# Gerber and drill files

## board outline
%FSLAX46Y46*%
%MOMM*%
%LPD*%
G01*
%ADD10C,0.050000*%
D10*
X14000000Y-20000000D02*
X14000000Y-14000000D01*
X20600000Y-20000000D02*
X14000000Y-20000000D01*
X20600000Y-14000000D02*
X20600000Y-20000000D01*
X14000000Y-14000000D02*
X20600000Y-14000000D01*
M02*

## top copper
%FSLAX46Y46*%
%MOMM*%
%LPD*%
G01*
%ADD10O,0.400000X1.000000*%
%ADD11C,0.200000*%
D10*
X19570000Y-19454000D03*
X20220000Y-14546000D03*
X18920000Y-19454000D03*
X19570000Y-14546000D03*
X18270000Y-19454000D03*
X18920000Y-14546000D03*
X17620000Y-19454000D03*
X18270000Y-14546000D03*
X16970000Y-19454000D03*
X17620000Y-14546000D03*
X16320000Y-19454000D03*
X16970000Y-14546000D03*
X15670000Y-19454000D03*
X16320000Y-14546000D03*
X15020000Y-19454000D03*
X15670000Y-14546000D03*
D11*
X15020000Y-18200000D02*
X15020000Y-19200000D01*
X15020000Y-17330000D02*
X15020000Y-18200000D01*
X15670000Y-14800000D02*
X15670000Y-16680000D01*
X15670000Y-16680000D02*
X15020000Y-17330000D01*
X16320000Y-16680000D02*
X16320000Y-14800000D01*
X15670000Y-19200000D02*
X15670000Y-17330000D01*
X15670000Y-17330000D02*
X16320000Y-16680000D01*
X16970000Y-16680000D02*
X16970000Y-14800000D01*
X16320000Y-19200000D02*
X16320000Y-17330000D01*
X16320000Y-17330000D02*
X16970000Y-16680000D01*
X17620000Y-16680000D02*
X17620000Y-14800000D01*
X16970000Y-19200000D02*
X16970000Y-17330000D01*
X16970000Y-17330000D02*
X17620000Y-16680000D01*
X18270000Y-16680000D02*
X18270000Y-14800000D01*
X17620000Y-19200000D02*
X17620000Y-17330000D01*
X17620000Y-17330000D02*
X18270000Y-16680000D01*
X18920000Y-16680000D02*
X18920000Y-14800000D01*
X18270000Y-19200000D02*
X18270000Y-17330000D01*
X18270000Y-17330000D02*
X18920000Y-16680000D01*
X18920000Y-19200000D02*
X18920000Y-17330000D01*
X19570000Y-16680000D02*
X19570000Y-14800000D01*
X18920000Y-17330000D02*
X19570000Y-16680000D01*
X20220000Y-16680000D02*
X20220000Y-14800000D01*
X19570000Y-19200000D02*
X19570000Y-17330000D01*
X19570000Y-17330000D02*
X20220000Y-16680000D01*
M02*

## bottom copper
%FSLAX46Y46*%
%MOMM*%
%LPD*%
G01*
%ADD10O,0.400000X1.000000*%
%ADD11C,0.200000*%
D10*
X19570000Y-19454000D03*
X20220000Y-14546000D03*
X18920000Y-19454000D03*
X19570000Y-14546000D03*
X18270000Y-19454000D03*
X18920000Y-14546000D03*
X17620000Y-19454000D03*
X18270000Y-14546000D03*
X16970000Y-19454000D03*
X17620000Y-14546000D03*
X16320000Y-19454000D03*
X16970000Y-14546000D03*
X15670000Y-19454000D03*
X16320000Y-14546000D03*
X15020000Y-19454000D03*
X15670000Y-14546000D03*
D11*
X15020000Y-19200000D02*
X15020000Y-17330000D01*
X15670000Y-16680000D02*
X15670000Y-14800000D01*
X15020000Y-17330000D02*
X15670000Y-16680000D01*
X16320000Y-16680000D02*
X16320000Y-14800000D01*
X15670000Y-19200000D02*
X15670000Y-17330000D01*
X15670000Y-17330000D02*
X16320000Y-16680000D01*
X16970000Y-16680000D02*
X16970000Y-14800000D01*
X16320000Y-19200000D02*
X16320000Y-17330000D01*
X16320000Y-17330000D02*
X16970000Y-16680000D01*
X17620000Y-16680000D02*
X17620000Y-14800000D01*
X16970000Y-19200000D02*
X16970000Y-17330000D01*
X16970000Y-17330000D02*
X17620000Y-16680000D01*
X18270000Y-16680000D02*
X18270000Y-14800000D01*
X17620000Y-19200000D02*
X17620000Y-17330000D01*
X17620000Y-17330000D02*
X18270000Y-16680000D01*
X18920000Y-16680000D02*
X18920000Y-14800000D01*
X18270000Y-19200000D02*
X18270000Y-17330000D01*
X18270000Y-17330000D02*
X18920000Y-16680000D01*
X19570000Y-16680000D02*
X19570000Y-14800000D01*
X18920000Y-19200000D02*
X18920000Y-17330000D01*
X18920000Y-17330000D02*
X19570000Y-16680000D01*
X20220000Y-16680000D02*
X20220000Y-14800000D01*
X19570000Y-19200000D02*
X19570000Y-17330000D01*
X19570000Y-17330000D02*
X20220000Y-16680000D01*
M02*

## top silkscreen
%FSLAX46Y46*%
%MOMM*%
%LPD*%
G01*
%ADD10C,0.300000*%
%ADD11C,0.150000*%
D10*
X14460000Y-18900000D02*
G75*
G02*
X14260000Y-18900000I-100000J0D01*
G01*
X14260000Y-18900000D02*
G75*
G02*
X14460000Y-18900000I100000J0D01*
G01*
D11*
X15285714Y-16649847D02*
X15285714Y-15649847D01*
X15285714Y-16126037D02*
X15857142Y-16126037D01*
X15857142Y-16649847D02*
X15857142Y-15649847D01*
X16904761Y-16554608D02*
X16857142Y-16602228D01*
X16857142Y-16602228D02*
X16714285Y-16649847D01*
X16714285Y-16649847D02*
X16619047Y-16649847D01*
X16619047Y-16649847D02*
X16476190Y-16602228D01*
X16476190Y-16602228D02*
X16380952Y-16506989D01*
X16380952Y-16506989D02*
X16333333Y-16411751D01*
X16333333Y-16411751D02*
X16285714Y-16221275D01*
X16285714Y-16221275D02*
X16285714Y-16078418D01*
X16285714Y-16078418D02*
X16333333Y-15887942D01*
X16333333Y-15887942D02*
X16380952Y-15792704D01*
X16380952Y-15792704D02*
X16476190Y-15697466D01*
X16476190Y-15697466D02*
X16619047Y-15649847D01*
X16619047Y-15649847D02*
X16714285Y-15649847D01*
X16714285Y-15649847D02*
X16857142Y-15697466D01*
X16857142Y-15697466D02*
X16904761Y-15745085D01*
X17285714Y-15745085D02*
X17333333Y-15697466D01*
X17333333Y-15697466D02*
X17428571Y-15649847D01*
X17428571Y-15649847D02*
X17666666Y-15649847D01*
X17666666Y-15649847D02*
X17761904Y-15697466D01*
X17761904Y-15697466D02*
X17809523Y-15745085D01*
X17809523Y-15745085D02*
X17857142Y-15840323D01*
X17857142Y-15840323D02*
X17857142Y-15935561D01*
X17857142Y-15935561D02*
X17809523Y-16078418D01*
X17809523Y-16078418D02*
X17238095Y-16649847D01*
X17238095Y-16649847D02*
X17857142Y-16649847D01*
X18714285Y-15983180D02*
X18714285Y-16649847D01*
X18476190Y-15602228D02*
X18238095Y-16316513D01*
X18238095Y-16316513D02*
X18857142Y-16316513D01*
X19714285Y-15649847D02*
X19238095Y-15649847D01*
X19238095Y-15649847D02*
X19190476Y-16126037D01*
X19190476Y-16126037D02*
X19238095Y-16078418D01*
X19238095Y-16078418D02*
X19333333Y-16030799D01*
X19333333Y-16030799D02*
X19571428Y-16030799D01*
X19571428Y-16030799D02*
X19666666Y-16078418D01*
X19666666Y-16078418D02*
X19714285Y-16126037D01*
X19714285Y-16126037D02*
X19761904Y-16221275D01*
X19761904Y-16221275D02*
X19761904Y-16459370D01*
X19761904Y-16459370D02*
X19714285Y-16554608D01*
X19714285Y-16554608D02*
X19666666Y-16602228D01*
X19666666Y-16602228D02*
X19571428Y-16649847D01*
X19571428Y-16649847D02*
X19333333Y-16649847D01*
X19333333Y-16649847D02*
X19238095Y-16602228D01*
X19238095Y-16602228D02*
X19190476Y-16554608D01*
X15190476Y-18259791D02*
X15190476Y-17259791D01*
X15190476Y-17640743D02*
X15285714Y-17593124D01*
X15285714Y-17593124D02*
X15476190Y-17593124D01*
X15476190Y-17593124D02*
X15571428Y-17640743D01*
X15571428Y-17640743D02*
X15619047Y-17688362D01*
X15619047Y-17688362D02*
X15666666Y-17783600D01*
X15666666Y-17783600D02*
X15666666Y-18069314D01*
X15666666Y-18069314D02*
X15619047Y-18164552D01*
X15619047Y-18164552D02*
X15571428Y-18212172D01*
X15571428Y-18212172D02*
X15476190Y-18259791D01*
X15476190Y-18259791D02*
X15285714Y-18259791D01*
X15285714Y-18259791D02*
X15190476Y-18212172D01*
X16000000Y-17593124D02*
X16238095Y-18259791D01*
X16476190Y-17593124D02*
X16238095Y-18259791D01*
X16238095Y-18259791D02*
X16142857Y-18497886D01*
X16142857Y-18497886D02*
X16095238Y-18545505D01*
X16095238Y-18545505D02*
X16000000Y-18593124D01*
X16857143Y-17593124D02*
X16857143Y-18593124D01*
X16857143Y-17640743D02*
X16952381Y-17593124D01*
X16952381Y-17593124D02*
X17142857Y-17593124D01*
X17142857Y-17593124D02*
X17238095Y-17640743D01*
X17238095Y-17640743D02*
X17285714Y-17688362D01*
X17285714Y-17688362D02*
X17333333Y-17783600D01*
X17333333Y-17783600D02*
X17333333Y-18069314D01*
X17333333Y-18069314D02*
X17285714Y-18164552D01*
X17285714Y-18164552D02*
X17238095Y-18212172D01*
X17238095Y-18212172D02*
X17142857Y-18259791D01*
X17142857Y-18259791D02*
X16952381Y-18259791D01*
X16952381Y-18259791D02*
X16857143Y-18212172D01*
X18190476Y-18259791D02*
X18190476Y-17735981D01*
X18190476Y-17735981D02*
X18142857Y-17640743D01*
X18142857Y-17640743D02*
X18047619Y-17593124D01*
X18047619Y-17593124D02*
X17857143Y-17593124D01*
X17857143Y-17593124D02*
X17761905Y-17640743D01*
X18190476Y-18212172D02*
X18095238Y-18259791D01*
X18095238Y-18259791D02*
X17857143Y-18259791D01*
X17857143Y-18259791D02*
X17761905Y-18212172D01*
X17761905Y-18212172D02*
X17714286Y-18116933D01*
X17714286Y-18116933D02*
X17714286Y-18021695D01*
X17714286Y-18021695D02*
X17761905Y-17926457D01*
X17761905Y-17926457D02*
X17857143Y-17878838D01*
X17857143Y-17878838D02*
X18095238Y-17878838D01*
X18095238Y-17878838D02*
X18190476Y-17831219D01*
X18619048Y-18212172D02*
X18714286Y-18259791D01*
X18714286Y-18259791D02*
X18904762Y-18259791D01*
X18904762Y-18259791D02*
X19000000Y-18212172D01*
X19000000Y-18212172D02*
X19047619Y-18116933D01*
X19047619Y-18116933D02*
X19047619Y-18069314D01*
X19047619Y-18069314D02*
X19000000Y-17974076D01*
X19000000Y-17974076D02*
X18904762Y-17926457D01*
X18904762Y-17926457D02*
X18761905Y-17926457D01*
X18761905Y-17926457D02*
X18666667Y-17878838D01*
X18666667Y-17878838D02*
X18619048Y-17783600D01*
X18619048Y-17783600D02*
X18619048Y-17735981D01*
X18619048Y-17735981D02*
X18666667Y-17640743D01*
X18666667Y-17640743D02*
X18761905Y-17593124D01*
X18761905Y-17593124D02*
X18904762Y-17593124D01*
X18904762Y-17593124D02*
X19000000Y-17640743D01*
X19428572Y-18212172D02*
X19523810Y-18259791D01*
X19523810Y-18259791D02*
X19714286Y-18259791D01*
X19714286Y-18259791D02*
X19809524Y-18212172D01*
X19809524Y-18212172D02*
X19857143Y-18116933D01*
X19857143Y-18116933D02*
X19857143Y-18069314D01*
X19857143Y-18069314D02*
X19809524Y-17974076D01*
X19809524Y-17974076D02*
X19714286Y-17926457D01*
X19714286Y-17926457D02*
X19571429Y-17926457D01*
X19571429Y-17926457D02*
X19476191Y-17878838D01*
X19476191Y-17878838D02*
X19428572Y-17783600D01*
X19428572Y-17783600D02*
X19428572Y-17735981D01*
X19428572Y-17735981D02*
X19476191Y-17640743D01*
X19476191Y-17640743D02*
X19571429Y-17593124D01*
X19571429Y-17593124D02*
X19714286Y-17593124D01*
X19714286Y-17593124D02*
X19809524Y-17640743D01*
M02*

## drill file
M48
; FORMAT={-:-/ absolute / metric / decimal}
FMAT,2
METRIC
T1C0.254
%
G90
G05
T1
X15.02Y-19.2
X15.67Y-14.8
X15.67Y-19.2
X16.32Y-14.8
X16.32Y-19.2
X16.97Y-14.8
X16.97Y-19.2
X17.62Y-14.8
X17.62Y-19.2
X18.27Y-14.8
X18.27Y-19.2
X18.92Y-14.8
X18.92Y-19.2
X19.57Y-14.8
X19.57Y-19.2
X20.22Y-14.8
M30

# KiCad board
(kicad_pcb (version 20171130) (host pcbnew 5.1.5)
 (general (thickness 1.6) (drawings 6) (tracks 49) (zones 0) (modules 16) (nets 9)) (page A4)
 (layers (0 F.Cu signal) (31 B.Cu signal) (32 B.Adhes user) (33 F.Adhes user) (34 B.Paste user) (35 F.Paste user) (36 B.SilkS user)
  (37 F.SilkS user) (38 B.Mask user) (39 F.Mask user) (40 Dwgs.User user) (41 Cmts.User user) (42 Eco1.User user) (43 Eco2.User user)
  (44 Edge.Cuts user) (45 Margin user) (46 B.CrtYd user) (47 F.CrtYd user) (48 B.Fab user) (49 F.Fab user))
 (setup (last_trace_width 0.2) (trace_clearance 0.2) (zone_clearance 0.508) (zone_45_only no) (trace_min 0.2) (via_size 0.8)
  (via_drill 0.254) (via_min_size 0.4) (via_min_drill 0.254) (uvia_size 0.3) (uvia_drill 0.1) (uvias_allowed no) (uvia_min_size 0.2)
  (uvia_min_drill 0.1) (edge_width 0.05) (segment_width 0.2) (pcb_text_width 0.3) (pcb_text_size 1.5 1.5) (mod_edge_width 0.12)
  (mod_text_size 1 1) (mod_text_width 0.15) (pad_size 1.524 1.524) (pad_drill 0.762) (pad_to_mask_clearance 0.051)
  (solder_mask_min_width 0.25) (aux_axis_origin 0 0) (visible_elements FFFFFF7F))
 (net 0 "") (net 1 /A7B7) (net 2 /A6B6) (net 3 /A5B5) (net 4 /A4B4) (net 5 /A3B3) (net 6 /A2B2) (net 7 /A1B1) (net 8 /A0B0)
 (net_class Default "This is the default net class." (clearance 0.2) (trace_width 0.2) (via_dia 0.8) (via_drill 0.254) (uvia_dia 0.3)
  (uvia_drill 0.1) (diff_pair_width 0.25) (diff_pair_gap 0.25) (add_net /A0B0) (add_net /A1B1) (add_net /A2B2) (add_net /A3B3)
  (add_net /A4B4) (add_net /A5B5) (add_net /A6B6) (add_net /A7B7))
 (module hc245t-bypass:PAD (layer F.Cu) (at 19.57 19.2)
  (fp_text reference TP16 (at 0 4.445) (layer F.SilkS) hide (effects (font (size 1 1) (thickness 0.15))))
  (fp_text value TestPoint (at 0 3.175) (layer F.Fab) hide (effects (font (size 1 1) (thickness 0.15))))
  (pad 1 thru_hole oval (at 0 0) (size 0.4 1) (drill 0.254 (offset 0 0.254)) (layers *.Cu *.Mask) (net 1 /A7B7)))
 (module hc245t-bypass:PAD (layer F.Cu) (at 20.22 14.8 180)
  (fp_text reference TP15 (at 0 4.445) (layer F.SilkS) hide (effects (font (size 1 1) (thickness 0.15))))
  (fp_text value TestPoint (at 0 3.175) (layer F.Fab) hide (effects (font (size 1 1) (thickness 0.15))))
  (pad 1 thru_hole oval (at 0 0 180) (size 0.4 1) (drill 0.254 (offset 0 0.254)) (layers *.Cu *.Mask) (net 1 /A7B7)))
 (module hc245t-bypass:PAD (layer F.Cu) (at 18.92 19.2)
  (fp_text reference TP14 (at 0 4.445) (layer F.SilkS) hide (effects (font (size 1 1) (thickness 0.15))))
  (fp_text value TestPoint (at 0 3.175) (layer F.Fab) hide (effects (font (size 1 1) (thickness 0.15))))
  (pad 1 thru_hole oval (at 0 0) (size 0.4 1) (drill 0.254 (offset 0 0.254)) (layers *.Cu *.Mask) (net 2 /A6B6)))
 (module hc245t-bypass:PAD (layer F.Cu) (at 19.57 14.8 180)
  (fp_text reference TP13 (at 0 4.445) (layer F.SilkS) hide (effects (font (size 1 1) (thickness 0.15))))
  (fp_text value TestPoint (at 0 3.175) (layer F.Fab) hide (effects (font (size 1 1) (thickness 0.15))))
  (pad 1 thru_hole oval (at 0 0 180) (size 0.4 1) (drill 0.254 (offset 0 0.254)) (layers *.Cu *.Mask) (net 2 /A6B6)))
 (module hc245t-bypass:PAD (layer F.Cu) (at 18.27 19.2)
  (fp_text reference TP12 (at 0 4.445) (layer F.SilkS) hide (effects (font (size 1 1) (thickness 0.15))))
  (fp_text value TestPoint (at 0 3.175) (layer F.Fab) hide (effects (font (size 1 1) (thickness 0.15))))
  (pad 1 thru_hole oval (at 0 0) (size 0.4 1) (drill 0.254 (offset 0 0.254)) (layers *.Cu *.Mask) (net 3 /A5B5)))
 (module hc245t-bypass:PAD (layer F.Cu) (at 18.92 14.8 180)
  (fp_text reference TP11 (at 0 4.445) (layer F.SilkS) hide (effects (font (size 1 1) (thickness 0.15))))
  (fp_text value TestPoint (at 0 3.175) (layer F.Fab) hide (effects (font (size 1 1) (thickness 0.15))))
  (pad 1 thru_hole oval (at 0 0 180) (size 0.4 1) (drill 0.254 (offset 0 0.254)) (layers *.Cu *.Mask) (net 3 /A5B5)))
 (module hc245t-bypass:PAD (layer F.Cu) (at 17.62 19.2)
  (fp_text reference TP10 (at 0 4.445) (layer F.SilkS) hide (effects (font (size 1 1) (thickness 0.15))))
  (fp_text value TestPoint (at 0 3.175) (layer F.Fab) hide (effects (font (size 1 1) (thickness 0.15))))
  (pad 1 thru_hole oval (at 0 0) (size 0.4 1) (drill 0.254 (offset 0 0.254)) (layers *.Cu *.Mask) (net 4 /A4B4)))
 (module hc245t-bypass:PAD (layer F.Cu) (at 18.27 14.8 180)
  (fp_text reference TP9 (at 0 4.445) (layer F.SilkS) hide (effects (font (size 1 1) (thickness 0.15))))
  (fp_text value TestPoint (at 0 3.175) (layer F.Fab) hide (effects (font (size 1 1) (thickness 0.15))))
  (pad 1 thru_hole oval (at 0 0 180) (size 0.4 1) (drill 0.254 (offset 0 0.254)) (layers *.Cu *.Mask) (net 4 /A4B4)))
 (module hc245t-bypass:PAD (layer F.Cu) (at 16.97 19.2)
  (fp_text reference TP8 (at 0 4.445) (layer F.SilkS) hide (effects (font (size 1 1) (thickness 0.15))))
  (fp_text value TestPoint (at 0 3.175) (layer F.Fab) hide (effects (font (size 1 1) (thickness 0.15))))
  (pad 1 thru_hole oval (at 0 0) (size 0.4 1) (drill 0.254 (offset 0 0.254)) (layers *.Cu *.Mask) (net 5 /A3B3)))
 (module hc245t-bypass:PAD (layer F.Cu) (at 17.62 14.8 180)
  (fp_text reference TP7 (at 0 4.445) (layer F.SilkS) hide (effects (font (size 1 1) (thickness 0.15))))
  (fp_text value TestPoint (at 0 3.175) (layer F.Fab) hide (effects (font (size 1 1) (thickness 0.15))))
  (pad 1 thru_hole oval (at 0 0 180) (size 0.4 1) (drill 0.254 (offset 0 0.254)) (layers *.Cu *.Mask) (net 5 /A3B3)))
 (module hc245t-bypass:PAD (layer F.Cu) (at 16.32 19.2)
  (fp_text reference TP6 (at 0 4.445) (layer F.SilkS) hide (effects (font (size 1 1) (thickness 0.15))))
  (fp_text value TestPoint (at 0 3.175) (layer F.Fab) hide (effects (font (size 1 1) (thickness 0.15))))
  (pad 1 thru_hole oval (at 0 0) (size 0.4 1) (drill 0.254 (offset 0 0.254)) (layers *.Cu *.Mask) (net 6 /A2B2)))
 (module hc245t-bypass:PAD (layer F.Cu) (at 16.97 14.8 180)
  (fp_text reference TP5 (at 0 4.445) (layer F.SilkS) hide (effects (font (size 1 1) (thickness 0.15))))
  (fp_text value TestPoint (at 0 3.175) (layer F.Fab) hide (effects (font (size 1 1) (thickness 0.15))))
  (pad 1 thru_hole oval (at 0 0 180) (size 0.4 1) (drill 0.254 (offset 0 0.254)) (layers *.Cu *.Mask) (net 6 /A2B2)))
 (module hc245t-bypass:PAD (layer F.Cu) (at 15.67 19.2)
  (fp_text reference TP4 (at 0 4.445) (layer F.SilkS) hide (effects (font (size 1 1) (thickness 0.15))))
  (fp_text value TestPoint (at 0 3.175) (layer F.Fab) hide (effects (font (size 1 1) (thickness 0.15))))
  (pad 1 thru_hole oval (at 0 0) (size 0.4 1) (drill 0.254 (offset 0 0.254)) (layers *.Cu *.Mask) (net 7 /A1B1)))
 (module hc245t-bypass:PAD (layer F.Cu) (at 16.32 14.8 180)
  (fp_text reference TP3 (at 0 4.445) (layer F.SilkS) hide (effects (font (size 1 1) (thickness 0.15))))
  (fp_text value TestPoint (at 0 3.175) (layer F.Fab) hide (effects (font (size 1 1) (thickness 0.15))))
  (pad 1 thru_hole oval (at 0 0 180) (size 0.4 1) (drill 0.254 (offset 0 0.254)) (layers *.Cu *.Mask) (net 7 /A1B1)))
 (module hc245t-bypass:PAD (layer F.Cu) (at 15.02 19.2)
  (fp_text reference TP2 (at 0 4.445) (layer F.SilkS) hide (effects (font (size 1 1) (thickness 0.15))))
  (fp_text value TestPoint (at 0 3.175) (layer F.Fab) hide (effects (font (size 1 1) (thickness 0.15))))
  (pad 1 thru_hole oval (at 0 0) (size 0.4 1) (drill 0.254 (offset 0 0.254)) (layers *.Cu *.Mask) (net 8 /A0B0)))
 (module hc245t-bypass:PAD (layer F.Cu) (at 15.67 14.8 180)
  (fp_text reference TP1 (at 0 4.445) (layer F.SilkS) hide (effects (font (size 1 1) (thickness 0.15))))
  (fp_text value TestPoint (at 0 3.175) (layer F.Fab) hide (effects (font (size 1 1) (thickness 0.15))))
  (pad 1 thru_hole oval (at 0 0 180) (size 0.4 1) (drill 0.254 (offset 0 0.254)) (layers *.Cu *.Mask) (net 8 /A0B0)))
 (gr_circle (center 14.36 18.9) (end 14.46 18.9) (layer F.SilkS) (width 0.3))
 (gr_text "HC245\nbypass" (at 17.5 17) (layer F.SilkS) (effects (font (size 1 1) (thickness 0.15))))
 (gr_line (start 14 20) (end 14 14) (layer Edge.Cuts) (width 0.05))
 (gr_line (start 20.6 20) (end 14 20) (layer Edge.Cuts) (width 0.05))
 (gr_line (start 20.6 14) (end 20.6 20) (layer Edge.Cuts) (width 0.05))
 (gr_line (start 14 14) (end 20.6 14) (layer Edge.Cuts) (width 0.05))
 (segment (start 15.02 19.2) (end 15.02 17.33) (width 0.2) (layer B.Cu) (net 8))
 (segment (start 15.67 16.68) (end 15.67 14.8) (width 0.2) (layer B.Cu) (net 8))
 (segment (start 15.02 17.33) (end 15.67 16.68) (width 0.2) (layer B.Cu) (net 8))
 (segment (start 15.02 18.2) (end 15.02 19.2) (width 0.2) (layer F.Cu) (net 8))
 (segment (start 15.02 17.33) (end 15.02 18.2) (width 0.2) (layer F.Cu) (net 8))
 (segment (start 15.67 14.8) (end 15.67 16.68) (width 0.2) (layer F.Cu) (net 8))
 (segment (start 15.67 16.68) (end 15.02 17.33) (width 0.2) (layer F.Cu) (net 8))
 (segment (start 16.32 16.68) (end 16.32 14.8) (width 0.2) (layer B.Cu) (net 7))
 (segment (start 15.67 19.2) (end 15.67 17.33) (width 0.2) (layer B.Cu) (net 7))
 (segment (start 15.67 17.33) (end 16.32 16.68) (width 0.2) (layer B.Cu) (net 7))
 (segment (start 16.32 16.68) (end 16.32 14.8) (width 0.2) (layer F.Cu) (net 7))
 (segment (start 15.67 19.2) (end 15.67 17.33) (width 0.2) (layer F.Cu) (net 7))
 (segment (start 15.67 17.33) (end 16.32 16.68) (width 0.2) (layer F.Cu) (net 7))
 (segment (start 16.97 16.68) (end 16.97 14.8) (width 0.2) (layer B.Cu) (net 6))
 (segment (start 16.32 19.2) (end 16.32 17.33) (width 0.2) (layer B.Cu) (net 6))
 (segment (start 16.32 17.33) (end 16.97 16.68) (width 0.2) (layer B.Cu) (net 6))
 (segment (start 16.97 16.68) (end 16.97 14.8) (width 0.2) (layer F.Cu) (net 6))
 (segment (start 16.32 19.2) (end 16.32 17.33) (width 0.2) (layer F.Cu) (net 6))
 (segment (start 16.32 17.33) (end 16.97 16.68) (width 0.2) (layer F.Cu) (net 6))
 (segment (start 17.62 16.68) (end 17.62 14.8) (width 0.2) (layer B.Cu) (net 5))
 (segment (start 16.97 19.2) (end 16.97 17.33) (width 0.2) (layer B.Cu) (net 5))
 (segment (start 16.97 17.33) (end 17.62 16.68) (width 0.2) (layer B.Cu) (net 5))
 (segment (start 17.62 16.68) (end 17.62 14.8) (width 0.2) (layer F.Cu) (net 5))
 (segment (start 16.97 19.2) (end 16.97 17.33) (width 0.2) (layer F.Cu) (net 5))
 (segment (start 16.97 17.33) (end 17.62 16.68) (width 0.2) (layer F.Cu) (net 5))
 (segment (start 18.27 16.68) (end 18.27 14.8) (width 0.2) (layer B.Cu) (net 4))
 (segment (start 17.62 19.2) (end 17.62 17.33) (width 0.2) (layer B.Cu) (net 4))
 (segment (start 17.62 17.33) (end 18.27 16.68) (width 0.2) (layer B.Cu) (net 4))
 (segment (start 18.27 16.68) (end 18.27 14.8) (width 0.2) (layer F.Cu) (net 4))
 (segment (start 17.62 19.2) (end 17.62 17.33) (width 0.2) (layer F.Cu) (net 4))
 (segment (start 17.62 17.33) (end 18.27 16.68) (width 0.2) (layer F.Cu) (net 4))
 (segment (start 18.92 16.68) (end 18.92 14.8) (width 0.2) (layer B.Cu) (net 3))
 (segment (start 18.27 19.2) (end 18.27 17.33) (width 0.2) (layer B.Cu) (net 3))
 (segment (start 18.27 17.33) (end 18.92 16.68) (width 0.2) (layer B.Cu) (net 3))
 (segment (start 18.92 16.68) (end 18.92 14.8) (width 0.2) (layer F.Cu) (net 3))
 (segment (start 18.27 19.2) (end 18.27 17.33) (width 0.2) (layer F.Cu) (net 3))
 (segment (start 18.27 17.33) (end 18.92 16.68) (width 0.2) (layer F.Cu) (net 3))
 (segment (start 19.57 16.68) (end 19.57 14.8) (width 0.2) (layer B.Cu) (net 2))
 (segment (start 18.92 19.2) (end 18.92 17.33) (width 0.2) (layer B.Cu) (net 2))
 (segment (start 18.92 17.33) (end 19.57 16.68) (width 0.2) (layer B.Cu) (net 2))
 (segment (start 18.92 19.2) (end 18.92 17.33) (width 0.2) (layer F.Cu) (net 2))
 (segment (start 19.57 16.68) (end 19.57 14.8) (width 0.2) (layer F.Cu) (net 2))
 (segment (start 18.92 17.33) (end 19.57 16.68) (width 0.2) (layer F.Cu) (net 2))
 (segment (start 20.22 16.68) (end 20.22 14.8) (width 0.2) (layer B.Cu) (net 1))
 (segment (start 19.57 19.2) (end 19.57 17.33) (width 0.2) (layer B.Cu) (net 1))
 (segment (start 19.57 17.33) (end 20.22 16.68) (width 0.2) (layer B.Cu) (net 1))
 (segment (start 20.22 16.68) (end 20.22 14.8) (width 0.2) (layer F.Cu) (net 1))
 (segment (start 19.57 19.2) (end 19.57 17.33) (width 0.2) (layer F.Cu) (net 1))
 (segment (start 19.57 17.33) (end 20.22 16.68) (width 0.2) (layer F.Cu) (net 1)))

